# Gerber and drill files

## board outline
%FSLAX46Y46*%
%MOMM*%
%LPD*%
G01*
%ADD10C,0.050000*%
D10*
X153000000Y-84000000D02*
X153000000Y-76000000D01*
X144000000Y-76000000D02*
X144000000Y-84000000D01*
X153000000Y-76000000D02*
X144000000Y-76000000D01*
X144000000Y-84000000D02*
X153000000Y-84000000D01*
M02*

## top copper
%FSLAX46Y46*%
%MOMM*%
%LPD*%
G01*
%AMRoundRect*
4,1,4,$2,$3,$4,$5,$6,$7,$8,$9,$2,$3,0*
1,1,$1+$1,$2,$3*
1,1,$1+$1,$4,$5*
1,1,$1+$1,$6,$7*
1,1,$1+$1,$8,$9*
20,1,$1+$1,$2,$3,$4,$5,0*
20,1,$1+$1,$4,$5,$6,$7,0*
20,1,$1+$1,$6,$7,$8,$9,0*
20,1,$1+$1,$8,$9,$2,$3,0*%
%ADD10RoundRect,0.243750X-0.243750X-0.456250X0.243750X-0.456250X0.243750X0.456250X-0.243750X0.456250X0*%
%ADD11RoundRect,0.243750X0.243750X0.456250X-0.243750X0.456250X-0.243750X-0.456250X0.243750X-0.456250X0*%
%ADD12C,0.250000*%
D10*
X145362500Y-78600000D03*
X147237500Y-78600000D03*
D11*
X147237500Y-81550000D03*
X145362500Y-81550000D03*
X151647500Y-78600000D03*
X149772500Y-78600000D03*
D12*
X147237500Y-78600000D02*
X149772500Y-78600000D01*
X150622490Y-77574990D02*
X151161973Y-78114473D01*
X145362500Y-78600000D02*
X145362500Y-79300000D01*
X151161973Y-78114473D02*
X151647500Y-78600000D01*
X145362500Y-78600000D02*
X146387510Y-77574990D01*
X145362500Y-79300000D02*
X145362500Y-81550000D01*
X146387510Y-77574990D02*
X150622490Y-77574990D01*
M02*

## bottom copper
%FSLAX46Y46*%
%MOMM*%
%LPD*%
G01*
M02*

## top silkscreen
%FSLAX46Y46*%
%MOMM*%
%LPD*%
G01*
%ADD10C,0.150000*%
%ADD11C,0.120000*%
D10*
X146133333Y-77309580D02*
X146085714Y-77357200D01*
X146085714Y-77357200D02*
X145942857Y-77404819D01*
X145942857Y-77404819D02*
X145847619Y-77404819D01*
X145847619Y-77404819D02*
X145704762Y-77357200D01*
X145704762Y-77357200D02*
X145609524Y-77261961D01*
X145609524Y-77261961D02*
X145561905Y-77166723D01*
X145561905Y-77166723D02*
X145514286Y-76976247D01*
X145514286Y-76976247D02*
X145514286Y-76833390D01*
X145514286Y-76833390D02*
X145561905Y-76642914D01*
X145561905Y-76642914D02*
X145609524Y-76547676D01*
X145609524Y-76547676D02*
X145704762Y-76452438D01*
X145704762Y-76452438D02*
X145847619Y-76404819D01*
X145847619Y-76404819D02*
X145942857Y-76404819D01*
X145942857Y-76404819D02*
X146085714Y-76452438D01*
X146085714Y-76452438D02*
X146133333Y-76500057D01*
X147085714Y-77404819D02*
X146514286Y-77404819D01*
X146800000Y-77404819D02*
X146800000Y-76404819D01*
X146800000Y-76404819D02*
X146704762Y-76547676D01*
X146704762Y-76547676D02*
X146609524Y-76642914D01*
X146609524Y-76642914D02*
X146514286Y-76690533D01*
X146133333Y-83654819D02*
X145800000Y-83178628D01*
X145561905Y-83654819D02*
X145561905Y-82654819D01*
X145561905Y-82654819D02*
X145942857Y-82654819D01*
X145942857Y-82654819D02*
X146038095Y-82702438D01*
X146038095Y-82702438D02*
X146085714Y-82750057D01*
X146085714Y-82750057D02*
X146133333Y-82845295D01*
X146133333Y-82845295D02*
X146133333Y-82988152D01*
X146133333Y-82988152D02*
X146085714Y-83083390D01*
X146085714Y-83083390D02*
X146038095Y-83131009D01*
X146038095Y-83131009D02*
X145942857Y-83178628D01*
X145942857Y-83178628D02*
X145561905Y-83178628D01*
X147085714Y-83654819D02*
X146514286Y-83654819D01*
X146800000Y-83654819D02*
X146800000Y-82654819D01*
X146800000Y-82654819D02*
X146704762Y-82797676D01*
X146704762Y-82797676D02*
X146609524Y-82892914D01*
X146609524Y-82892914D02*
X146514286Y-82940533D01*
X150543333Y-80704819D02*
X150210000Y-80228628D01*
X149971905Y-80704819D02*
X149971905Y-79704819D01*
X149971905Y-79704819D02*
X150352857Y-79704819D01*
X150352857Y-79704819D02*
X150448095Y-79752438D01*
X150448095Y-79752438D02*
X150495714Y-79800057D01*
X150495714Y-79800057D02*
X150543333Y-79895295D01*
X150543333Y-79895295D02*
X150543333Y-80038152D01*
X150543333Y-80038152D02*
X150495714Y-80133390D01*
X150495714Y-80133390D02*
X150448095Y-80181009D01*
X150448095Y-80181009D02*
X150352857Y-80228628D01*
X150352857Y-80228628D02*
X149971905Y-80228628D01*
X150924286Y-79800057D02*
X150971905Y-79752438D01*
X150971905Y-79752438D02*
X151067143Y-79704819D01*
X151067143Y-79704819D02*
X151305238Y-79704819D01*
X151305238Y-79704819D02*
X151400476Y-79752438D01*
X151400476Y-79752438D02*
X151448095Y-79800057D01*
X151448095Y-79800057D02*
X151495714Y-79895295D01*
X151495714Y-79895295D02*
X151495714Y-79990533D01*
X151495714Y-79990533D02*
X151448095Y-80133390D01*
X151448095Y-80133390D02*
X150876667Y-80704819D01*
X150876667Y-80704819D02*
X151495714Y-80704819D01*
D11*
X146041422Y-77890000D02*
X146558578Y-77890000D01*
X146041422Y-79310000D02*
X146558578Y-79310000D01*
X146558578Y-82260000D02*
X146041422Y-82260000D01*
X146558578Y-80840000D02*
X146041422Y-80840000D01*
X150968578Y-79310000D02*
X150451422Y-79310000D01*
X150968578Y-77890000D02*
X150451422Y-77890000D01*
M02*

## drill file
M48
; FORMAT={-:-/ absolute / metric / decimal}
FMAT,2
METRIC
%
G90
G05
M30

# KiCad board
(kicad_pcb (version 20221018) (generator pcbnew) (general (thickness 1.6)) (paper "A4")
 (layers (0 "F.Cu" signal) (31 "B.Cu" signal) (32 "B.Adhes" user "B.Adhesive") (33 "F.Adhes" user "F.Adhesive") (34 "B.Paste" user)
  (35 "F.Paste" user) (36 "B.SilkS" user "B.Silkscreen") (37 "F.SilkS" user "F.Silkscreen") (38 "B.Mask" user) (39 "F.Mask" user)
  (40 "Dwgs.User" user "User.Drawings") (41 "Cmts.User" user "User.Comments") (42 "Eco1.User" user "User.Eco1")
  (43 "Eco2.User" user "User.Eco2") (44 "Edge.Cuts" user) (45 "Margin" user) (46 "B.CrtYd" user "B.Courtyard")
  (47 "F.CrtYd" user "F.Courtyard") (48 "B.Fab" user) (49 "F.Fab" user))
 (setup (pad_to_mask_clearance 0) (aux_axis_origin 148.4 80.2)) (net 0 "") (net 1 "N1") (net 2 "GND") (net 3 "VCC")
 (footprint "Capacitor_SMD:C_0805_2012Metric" (layer "F.Cu") (at 146.3 78.6)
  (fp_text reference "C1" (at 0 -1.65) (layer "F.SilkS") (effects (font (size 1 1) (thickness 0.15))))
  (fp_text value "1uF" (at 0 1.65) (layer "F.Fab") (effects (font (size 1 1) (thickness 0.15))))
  (fp_line (start -0.258578 -0.71) (end 0.258578 -0.71) (stroke (width 0.12) (type solid)) (layer "F.SilkS"))
  (fp_line (start -0.258578 0.71) (end 0.258578 0.71) (stroke (width 0.12) (type solid)) (layer "F.SilkS"))
  (pad "1" smd roundrect (at -0.9375 0) (size 0.975 1.4) (layers "F.Cu" "F.Paste" "F.Mask") (roundrect_rratio 0.25) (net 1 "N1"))
  (pad "2" smd roundrect (at 0.9375 0) (size 0.975 1.4) (layers "F.Cu" "F.Paste" "F.Mask") (roundrect_rratio 0.25) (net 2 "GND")))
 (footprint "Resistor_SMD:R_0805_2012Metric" (layer "F.Cu") (at 146.3 81.55 180)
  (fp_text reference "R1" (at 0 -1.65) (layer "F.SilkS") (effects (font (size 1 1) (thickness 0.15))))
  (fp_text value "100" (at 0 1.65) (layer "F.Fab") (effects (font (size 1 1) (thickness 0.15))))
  (fp_line (start -0.258578 -0.71) (end 0.258578 -0.71) (stroke (width 0.12) (type solid)) (layer "F.SilkS"))
  (fp_line (start -0.258578 0.71) (end 0.258578 0.71) (stroke (width 0.12) (type solid)) (layer "F.SilkS"))
  (pad "1" smd roundrect (at -0.9375 0 180) (size 0.975 1.4) (layers "F.Cu" "F.Paste" "F.Mask") (roundrect_rratio 0.25) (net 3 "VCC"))
  (pad "2" smd roundrect (at 0.9375 0 180) (size 0.975 1.4) (layers "F.Cu" "F.Paste" "F.Mask") (roundrect_rratio 0.25) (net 1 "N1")))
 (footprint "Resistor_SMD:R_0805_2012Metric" (layer "F.Cu") (at 150.71 78.6 180)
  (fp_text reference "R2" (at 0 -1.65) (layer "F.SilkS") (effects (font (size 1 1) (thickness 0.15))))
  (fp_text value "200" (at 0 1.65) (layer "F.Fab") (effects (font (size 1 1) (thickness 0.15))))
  (fp_line (start -0.258578 -0.71) (end 0.258578 -0.71) (stroke (width 0.12) (type solid)) (layer "F.SilkS"))
  (fp_line (start -0.258578 0.71) (end 0.258578 0.71) (stroke (width 0.12) (type solid)) (layer "F.SilkS"))
  (pad "1" smd roundrect (at -0.9375 0 180) (size 0.975 1.4) (layers "F.Cu" "F.Paste" "F.Mask") (roundrect_rratio 0.25) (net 1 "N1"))
  (pad "2" smd roundrect (at 0.9375 0 180) (size 0.975 1.4) (layers "F.Cu" "F.Paste" "F.Mask") (roundrect_rratio 0.25) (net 2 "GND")))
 (gr_line (start 153 84) (end 153 76) (stroke (width 0.05) (type solid)) (layer "Edge.Cuts"))
 (gr_line (start 144 76) (end 144 84) (stroke (width 0.05) (type solid)) (layer "Edge.Cuts"))
 (gr_line (start 153 76) (end 144 76) (stroke (width 0.05) (type solid)) (layer "Edge.Cuts"))
 (gr_line (start 144 84) (end 153 84) (stroke (width 0.05) (type solid)) (layer "Edge.Cuts"))
 (segment (start 147.2375 78.6) (end 149.7725 78.6) (width 0.25) (layer "F.Cu") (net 2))
 (segment (start 150.62249 77.57499) (end 151.161973 78.114473) (width 0.25) (layer "F.Cu") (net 1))
 (segment (start 145.3625 78.6) (end 145.3625 79.3) (width 0.25) (layer "F.Cu") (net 1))
 (segment (start 151.161973 78.114473) (end 151.6475 78.6) (width 0.25) (layer "F.Cu") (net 1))
 (segment (start 145.3625 78.6) (end 146.38751 77.57499) (width 0.25) (layer "F.Cu") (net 1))
 (segment (start 145.3625 79.3) (end 145.3625 81.55) (width 0.25) (layer "F.Cu") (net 1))
 (segment (start 146.38751 77.57499) (end 150.62249 77.57499) (width 0.25) (layer "F.Cu") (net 1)))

